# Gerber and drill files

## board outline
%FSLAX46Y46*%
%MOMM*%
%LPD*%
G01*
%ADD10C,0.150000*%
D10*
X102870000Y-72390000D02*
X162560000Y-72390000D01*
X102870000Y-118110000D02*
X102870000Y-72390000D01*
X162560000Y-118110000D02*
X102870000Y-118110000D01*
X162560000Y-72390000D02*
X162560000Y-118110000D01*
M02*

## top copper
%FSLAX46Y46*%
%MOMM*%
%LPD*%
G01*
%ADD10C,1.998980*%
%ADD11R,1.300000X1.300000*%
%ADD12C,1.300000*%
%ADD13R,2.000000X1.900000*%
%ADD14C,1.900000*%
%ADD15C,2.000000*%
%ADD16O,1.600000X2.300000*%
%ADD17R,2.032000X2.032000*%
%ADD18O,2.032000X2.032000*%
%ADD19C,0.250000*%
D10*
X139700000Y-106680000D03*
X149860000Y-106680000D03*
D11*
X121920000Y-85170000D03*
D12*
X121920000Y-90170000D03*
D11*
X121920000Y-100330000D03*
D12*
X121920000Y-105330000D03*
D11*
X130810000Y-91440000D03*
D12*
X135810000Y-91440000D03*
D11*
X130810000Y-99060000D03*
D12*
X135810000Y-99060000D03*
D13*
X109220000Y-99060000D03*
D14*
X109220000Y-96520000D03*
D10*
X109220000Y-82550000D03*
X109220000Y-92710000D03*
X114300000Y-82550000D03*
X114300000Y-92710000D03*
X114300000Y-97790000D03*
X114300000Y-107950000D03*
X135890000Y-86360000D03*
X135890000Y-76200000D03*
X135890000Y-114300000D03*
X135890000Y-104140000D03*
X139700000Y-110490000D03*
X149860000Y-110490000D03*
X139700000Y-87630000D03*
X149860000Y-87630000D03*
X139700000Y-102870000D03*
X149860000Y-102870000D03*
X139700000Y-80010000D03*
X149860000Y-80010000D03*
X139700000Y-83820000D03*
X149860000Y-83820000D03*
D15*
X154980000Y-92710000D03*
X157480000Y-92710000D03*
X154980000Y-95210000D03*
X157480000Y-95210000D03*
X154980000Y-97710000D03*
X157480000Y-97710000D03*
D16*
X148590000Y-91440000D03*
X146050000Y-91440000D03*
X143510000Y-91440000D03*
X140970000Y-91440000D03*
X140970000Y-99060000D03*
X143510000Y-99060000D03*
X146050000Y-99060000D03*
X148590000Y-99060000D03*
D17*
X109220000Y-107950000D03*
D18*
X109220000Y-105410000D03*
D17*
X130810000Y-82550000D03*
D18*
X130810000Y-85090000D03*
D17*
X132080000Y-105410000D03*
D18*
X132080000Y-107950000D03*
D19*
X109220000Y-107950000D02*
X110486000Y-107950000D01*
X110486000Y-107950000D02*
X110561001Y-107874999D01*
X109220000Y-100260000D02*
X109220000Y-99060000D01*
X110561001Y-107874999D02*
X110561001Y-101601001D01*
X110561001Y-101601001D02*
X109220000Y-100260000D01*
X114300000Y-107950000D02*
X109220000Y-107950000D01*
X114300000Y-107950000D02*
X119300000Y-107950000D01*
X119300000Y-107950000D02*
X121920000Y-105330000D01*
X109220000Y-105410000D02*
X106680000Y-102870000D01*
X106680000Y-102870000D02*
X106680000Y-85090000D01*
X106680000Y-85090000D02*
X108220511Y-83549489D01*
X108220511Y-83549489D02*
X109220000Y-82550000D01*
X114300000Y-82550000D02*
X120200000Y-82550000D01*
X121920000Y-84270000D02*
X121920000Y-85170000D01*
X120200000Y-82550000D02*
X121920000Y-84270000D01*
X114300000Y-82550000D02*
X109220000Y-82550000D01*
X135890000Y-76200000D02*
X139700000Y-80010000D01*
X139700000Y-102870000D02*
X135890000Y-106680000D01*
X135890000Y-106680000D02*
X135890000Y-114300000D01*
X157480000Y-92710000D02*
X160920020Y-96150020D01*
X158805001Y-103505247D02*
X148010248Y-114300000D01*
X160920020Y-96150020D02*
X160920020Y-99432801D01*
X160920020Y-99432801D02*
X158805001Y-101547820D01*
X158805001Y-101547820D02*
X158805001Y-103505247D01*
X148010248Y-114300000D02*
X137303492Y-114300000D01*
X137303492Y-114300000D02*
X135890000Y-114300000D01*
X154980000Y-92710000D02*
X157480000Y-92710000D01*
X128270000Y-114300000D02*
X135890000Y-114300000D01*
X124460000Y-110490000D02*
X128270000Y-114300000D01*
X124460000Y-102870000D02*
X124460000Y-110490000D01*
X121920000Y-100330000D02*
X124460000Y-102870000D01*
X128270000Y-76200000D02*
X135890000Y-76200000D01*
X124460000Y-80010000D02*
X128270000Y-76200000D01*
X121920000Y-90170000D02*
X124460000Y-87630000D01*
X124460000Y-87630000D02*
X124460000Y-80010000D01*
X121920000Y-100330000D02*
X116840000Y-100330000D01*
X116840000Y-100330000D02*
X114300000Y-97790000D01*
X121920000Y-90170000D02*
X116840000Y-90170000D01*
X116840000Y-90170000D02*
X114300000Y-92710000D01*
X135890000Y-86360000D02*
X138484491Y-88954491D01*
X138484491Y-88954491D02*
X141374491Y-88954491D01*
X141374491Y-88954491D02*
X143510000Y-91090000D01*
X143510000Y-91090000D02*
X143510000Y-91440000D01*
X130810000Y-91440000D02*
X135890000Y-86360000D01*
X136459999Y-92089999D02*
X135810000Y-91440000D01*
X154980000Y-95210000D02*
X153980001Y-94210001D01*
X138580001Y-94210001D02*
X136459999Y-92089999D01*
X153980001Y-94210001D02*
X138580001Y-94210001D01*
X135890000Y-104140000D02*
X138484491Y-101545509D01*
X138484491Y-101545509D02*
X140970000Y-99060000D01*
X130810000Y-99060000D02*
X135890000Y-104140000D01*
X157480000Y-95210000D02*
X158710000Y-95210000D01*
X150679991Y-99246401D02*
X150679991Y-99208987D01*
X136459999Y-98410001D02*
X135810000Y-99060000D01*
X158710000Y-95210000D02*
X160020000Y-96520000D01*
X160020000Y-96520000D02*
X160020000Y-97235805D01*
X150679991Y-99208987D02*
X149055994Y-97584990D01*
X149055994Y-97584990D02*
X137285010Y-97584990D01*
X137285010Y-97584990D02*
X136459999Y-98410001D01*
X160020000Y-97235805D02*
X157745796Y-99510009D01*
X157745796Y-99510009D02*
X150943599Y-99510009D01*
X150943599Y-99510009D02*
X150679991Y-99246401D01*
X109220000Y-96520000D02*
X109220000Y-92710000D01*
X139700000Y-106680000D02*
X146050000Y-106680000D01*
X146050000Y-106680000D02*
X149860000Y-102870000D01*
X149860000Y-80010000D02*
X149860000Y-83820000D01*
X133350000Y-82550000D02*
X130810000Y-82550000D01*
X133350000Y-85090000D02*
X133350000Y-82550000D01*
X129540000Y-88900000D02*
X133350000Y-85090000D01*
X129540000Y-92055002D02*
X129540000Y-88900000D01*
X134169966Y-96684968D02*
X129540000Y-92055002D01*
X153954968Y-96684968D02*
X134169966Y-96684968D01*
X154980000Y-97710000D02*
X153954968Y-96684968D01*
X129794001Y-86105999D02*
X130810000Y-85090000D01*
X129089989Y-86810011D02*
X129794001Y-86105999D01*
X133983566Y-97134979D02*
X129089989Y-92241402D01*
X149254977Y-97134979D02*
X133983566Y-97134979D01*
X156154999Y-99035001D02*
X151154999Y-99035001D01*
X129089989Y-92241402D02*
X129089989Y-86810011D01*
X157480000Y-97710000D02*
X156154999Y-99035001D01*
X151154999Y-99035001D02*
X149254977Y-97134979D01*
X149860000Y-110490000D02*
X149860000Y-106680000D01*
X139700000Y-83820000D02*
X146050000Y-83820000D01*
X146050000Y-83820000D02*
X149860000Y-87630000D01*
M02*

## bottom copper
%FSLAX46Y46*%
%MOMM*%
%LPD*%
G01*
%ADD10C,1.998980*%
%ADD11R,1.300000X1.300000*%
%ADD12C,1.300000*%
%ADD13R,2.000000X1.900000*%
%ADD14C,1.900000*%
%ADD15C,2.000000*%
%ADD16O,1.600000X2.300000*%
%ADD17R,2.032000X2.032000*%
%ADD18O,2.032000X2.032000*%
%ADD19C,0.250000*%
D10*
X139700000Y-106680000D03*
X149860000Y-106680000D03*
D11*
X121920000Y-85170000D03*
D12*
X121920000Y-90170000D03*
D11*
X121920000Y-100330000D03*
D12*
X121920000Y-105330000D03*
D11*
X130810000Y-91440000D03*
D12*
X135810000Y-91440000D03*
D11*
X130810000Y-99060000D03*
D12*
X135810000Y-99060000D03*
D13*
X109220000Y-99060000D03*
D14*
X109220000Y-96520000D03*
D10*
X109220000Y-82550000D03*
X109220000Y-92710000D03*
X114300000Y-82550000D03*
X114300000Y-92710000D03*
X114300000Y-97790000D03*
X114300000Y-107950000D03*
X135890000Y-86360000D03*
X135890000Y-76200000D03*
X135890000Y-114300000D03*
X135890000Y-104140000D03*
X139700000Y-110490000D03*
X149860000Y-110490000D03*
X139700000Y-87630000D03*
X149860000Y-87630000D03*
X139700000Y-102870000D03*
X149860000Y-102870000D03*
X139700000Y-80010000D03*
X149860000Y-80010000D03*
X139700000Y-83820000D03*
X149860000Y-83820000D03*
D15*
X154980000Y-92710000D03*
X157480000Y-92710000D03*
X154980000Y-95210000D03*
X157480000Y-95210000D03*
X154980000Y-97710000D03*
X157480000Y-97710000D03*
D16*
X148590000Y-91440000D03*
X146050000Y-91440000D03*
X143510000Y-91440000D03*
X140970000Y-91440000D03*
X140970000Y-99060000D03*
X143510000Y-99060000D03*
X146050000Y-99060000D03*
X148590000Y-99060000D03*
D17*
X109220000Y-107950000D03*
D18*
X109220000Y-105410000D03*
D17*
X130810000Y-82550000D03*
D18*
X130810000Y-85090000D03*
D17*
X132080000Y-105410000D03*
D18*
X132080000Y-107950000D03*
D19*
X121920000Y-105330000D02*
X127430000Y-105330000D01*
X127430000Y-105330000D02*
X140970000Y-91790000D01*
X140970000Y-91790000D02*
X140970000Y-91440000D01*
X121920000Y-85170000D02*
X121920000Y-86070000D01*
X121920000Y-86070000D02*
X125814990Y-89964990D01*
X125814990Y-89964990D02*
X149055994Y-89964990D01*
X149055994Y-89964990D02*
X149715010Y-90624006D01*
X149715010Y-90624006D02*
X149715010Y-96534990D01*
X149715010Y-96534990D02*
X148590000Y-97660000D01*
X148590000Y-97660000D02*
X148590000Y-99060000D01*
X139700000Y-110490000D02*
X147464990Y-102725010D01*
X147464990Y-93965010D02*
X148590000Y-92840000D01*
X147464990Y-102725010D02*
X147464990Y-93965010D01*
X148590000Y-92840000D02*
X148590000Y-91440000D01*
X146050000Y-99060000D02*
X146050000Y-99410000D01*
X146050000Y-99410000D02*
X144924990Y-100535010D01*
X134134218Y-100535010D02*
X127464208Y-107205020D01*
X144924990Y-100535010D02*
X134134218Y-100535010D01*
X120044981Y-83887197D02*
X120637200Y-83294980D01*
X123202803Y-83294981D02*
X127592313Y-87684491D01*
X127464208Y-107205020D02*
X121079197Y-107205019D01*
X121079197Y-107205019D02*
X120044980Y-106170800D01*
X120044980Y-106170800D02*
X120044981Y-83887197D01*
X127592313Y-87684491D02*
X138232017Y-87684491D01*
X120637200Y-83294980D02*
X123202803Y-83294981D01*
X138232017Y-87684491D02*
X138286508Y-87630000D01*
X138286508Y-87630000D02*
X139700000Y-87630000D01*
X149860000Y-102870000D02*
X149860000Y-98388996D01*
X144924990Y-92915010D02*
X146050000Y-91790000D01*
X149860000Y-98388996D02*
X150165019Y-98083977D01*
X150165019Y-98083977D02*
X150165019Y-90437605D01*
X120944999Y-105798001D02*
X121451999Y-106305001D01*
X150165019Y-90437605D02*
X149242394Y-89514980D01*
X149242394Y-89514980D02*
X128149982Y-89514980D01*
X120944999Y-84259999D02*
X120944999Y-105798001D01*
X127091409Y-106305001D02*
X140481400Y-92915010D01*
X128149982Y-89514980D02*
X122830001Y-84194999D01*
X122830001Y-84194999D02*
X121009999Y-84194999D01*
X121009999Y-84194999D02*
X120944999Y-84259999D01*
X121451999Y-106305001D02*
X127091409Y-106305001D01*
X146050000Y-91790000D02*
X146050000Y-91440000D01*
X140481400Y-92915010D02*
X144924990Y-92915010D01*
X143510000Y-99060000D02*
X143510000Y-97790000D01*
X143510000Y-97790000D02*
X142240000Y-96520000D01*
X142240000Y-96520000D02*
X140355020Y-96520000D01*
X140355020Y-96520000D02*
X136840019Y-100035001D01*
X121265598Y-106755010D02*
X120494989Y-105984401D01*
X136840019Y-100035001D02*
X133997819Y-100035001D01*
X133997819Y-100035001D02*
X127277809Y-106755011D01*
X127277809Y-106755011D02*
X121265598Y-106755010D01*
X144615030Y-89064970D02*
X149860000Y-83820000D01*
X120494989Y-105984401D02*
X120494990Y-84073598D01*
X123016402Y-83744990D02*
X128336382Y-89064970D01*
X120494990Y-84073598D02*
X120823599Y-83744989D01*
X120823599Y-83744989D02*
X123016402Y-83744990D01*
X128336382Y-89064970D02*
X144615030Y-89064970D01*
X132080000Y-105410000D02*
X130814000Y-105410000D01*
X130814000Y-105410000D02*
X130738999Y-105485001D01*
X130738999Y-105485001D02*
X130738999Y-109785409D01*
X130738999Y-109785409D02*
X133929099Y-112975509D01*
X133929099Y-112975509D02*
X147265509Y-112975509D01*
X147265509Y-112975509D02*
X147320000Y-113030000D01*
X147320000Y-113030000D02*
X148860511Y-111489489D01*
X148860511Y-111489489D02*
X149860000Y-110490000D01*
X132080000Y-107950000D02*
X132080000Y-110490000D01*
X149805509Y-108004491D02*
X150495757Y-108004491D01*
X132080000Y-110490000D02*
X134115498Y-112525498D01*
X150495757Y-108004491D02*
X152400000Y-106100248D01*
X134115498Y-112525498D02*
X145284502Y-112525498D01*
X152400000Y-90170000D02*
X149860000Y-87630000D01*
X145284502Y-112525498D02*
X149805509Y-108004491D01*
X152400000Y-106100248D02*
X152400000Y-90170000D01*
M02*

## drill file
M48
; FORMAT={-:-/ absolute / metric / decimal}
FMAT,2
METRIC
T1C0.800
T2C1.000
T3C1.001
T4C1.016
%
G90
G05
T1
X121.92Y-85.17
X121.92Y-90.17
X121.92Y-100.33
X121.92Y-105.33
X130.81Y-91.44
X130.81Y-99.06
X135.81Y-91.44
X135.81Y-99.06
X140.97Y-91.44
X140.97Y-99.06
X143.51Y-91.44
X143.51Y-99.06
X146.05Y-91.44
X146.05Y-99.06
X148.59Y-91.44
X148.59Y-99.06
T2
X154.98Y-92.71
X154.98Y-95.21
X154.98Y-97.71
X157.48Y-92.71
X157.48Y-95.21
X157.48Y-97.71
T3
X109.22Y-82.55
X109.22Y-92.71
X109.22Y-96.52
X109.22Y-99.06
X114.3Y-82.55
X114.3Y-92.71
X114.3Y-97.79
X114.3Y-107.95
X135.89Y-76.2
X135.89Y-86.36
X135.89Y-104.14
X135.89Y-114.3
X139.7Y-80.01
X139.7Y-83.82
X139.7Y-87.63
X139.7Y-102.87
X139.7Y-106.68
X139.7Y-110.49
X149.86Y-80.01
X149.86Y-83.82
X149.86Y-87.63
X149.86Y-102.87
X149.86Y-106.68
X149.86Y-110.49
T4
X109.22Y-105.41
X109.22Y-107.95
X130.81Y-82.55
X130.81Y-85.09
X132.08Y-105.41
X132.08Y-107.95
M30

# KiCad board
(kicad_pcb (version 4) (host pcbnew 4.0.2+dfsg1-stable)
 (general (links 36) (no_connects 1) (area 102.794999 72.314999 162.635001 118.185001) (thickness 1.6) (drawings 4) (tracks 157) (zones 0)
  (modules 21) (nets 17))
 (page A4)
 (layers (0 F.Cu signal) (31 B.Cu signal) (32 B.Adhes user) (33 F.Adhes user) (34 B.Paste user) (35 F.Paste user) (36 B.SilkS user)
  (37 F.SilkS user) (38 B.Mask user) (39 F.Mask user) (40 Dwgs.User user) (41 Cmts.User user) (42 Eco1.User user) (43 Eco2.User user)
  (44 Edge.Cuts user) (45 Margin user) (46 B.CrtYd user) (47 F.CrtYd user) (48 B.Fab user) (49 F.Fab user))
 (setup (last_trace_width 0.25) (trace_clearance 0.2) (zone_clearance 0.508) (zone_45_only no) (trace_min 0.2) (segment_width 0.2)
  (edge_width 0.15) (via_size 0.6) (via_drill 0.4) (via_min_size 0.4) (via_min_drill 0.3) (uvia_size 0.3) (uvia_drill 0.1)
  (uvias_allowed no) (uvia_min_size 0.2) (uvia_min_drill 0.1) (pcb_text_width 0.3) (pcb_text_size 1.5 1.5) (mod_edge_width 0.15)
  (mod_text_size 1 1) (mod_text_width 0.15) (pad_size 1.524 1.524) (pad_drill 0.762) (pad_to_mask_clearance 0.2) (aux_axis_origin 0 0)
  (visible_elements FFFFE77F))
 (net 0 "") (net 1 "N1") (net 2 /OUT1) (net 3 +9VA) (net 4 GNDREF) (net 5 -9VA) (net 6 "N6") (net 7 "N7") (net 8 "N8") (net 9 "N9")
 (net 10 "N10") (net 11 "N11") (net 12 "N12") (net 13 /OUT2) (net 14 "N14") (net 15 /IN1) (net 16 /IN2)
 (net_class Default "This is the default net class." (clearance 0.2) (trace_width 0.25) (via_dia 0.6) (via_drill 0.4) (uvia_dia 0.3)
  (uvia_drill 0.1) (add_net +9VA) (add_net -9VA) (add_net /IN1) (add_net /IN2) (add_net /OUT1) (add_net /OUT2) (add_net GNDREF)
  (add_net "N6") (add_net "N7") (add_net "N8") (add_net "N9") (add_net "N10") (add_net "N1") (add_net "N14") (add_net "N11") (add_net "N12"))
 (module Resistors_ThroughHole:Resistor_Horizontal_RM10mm (layer F.Cu) (at 139.7 106.68)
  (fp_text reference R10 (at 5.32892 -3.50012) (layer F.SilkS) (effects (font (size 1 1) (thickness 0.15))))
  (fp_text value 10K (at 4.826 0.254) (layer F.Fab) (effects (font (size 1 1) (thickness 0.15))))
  (pad 1 thru_hole circle (at 0 0) (size 1.99898 1.99898) (drill 1.00076) (layers *.Cu *.SilkS *.Mask) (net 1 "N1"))
  (pad 2 thru_hole circle (at 10.16 0) (size 1.99898 1.99898) (drill 1.00076) (layers *.Cu *.SilkS *.Mask) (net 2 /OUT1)))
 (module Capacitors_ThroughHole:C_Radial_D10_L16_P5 (layer F.Cu) (at 121.92 85.17 270)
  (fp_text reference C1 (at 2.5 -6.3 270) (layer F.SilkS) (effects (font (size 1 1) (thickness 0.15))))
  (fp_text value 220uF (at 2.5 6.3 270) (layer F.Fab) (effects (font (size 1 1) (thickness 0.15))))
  (pad 1 thru_hole rect (at 0 0 270) (size 1.3 1.3) (drill 0.8) (layers *.Cu *.Mask F.SilkS) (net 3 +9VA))
  (pad 2 thru_hole circle (at 5 0 270) (size 1.3 1.3) (drill 0.8) (layers *.Cu *.Mask F.SilkS) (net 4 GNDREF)))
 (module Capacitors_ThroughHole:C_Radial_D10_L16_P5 (layer F.Cu) (at 121.92 100.33 270)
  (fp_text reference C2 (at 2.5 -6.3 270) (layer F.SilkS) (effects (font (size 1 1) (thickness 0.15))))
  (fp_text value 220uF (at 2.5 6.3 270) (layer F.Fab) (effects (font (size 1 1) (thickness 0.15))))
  (pad 1 thru_hole rect (at 0 0 270) (size 1.3 1.3) (drill 0.8) (layers *.Cu *.Mask F.SilkS) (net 4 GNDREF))
  (pad 2 thru_hole circle (at 5 0 270) (size 1.3 1.3) (drill 0.8) (layers *.Cu *.Mask F.SilkS) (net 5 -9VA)))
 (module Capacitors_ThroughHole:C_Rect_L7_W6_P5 (layer F.Cu) (at 130.81 91.44)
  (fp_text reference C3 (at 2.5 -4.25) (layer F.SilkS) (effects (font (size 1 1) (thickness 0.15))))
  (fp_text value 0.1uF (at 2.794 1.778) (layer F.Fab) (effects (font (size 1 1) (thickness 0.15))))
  (pad 1 thru_hole rect (at 0 0) (size 1.3 1.3) (drill 0.8) (layers *.Cu *.Mask F.SilkS) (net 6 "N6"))
  (pad 2 thru_hole circle (at 5 0) (size 1.3 1.3) (drill 0.8) (layers *.Cu *.Mask F.SilkS) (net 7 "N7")))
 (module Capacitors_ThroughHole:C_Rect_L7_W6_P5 (layer F.Cu) (at 130.81 99.06)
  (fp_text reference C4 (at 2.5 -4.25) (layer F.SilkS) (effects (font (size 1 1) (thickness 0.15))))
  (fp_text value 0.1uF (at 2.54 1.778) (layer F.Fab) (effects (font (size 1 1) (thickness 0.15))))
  (pad 1 thru_hole rect (at 0 0) (size 1.3 1.3) (drill 0.8) (layers *.Cu *.Mask F.SilkS) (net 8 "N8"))
  (pad 2 thru_hole circle (at 5 0) (size 1.3 1.3) (drill 0.8) (layers *.Cu *.Mask F.SilkS) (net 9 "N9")))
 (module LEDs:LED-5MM (layer F.Cu) (at 109.22 99.06 90)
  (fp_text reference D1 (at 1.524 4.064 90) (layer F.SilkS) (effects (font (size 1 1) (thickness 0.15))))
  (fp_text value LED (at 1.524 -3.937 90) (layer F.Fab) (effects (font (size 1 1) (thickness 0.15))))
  (pad 1 thru_hole rect (at 0 0 180) (size 2 1.9) (drill 1.00076) (layers *.Cu *.Mask F.SilkS) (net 5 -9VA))
  (pad 2 thru_hole circle (at 2.54 0 90) (size 1.9 1.9) (drill 1.00076) (layers *.Cu *.Mask F.SilkS) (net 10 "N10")))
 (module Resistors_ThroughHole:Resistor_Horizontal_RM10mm (layer F.Cu) (at 109.22 82.55 270)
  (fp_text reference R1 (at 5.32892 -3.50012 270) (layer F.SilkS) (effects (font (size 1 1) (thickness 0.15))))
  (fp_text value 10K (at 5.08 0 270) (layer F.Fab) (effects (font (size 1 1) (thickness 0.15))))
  (pad 1 thru_hole circle (at 0 0 270) (size 1.99898 1.99898) (drill 1.00076) (layers *.Cu *.SilkS *.Mask) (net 3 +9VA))
  (pad 2 thru_hole circle (at 10.16 0 270) (size 1.99898 1.99898) (drill 1.00076) (layers *.Cu *.SilkS *.Mask) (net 10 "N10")))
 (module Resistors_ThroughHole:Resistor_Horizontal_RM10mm (layer F.Cu) (at 114.3 82.55 270)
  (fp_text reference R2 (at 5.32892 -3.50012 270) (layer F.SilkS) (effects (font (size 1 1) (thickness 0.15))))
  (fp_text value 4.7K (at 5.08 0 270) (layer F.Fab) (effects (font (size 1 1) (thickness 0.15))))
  (pad 1 thru_hole circle (at 0 0 270) (size 1.99898 1.99898) (drill 1.00076) (layers *.Cu *.SilkS *.Mask) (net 3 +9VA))
  (pad 2 thru_hole circle (at 10.16 0 270) (size 1.99898 1.99898) (drill 1.00076) (layers *.Cu *.SilkS *.Mask) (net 4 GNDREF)))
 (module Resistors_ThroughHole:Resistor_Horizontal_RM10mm (layer F.Cu) (at 114.3 97.79 270)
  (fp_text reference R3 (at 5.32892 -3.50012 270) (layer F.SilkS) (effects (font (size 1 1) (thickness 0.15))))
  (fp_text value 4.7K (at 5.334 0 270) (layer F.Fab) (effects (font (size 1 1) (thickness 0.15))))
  (pad 1 thru_hole circle (at 0 0 270) (size 1.99898 1.99898) (drill 1.00076) (layers *.Cu *.SilkS *.Mask) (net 4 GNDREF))
  (pad 2 thru_hole circle (at 10.16 0 270) (size 1.99898 1.99898) (drill 1.00076) (layers *.Cu *.SilkS *.Mask) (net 5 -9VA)))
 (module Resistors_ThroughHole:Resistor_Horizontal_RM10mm (layer F.Cu) (at 135.89 86.36 90)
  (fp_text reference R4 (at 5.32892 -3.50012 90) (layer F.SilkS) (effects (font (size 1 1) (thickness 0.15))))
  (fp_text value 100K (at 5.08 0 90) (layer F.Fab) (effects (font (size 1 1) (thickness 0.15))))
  (pad 1 thru_hole circle (at 0 0 90) (size 1.99898 1.99898) (drill 1.00076) (layers *.Cu *.SilkS *.Mask) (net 6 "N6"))
  (pad 2 thru_hole circle (at 10.16 0 90) (size 1.99898 1.99898) (drill 1.00076) (layers *.Cu *.SilkS *.Mask) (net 4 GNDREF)))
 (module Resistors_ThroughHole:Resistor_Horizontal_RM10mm (layer F.Cu) (at 135.89 114.3 90)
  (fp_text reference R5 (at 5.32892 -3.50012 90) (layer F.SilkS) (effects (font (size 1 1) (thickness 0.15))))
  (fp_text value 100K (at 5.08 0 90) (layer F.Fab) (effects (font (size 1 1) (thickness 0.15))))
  (pad 1 thru_hole circle (at 0 0 90) (size 1.99898 1.99898) (drill 1.00076) (layers *.Cu *.SilkS *.Mask) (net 4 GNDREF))
  (pad 2 thru_hole circle (at 10.16 0 90) (size 1.99898 1.99898) (drill 1.00076) (layers *.Cu *.SilkS *.Mask) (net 8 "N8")))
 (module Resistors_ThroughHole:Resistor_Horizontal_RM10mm (layer F.Cu) (at 139.7 110.49)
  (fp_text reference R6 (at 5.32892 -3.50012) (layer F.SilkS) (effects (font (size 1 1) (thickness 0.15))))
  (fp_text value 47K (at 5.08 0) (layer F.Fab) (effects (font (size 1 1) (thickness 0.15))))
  (pad 1 thru_hole circle (at 0 0) (size 1.99898 1.99898) (drill 1.00076) (layers *.Cu *.SilkS *.Mask) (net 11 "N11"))
  (pad 2 thru_hole circle (at 10.16 0) (size 1.99898 1.99898) (drill 1.00076) (layers *.Cu *.SilkS *.Mask) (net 2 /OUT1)))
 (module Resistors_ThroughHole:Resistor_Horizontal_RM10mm (layer F.Cu) (at 139.7 87.63)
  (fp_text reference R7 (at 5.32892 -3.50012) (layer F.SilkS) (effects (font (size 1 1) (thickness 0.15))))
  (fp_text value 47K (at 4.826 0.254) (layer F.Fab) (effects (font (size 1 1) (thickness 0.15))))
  (pad 1 thru_hole circle (at 0 0) (size 1.99898 1.99898) (drill 1.00076) (layers *.Cu *.SilkS *.Mask) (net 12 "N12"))
  (pad 2 thru_hole circle (at 10.16 0) (size 1.99898 1.99898) (drill 1.00076) (layers *.Cu *.SilkS *.Mask) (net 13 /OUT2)))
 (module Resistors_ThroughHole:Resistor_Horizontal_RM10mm (layer F.Cu) (at 139.7 102.87)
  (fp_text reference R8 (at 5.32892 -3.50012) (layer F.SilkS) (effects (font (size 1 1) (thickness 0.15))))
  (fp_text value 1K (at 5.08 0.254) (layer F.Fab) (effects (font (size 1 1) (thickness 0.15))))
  (pad 1 thru_hole circle (at 0 0) (size 1.99898 1.99898) (drill 1.00076) (layers *.Cu *.SilkS *.Mask) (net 4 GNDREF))
  (pad 2 thru_hole circle (at 10.16 0) (size 1.99898 1.99898) (drill 1.00076) (layers *.Cu *.SilkS *.Mask) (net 1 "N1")))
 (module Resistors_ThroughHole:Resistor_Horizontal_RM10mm (layer F.Cu) (at 139.7 80.01)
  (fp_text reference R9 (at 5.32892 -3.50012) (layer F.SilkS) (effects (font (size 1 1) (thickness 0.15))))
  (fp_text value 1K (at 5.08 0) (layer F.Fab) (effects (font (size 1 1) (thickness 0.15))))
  (pad 1 thru_hole circle (at 0 0) (size 1.99898 1.99898) (drill 1.00076) (layers *.Cu *.SilkS *.Mask) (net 4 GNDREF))
  (pad 2 thru_hole circle (at 10.16 0) (size 1.99898 1.99898) (drill 1.00076) (layers *.Cu *.SilkS *.Mask) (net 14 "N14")))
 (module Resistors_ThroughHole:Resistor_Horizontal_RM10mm (layer F.Cu) (at 139.7 83.82)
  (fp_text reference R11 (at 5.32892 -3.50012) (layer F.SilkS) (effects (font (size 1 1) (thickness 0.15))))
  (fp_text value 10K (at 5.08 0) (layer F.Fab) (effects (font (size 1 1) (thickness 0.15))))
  (pad 1 thru_hole circle (at 0 0) (size 1.99898 1.99898) (drill 1.00076) (layers *.Cu *.SilkS *.Mask) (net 13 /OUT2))
  (pad 2 thru_hole circle (at 10.16 0) (size 1.99898 1.99898) (drill 1.00076) (layers *.Cu *.SilkS *.Mask) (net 14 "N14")))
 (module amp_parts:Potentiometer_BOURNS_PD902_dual (layer F.Cu) (at 162.48 95.21)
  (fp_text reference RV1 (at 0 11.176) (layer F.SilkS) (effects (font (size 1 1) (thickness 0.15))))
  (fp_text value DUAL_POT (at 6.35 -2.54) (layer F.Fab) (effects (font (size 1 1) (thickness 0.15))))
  (pad 3 thru_hole circle (at -7.5 -2.5) (size 2 2) (drill 1) (layers *.Cu *.Mask F.SilkS) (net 4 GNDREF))
  (pad 6 thru_hole circle (at -5 -2.5) (size 2 2) (drill 1) (layers *.Cu *.Mask F.SilkS) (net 4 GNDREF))
  (pad 2 thru_hole circle (at -7.5 0) (size 2 2) (drill 1) (layers *.Cu *.Mask F.SilkS) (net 7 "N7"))
  (pad 5 thru_hole circle (at -5 0) (size 2 2) (drill 1) (layers *.Cu *.Mask F.SilkS) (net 9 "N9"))
  (pad 1 thru_hole circle (at -7.5 2.5) (size 2 2) (drill 1) (layers *.Cu *.Mask F.SilkS) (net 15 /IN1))
  (pad 4 thru_hole circle (at -5 2.5) (size 2 2) (drill 1) (layers *.Cu *.Mask F.SilkS) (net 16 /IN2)))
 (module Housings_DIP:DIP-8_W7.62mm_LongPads (layer F.Cu) (at 148.59 91.44 270)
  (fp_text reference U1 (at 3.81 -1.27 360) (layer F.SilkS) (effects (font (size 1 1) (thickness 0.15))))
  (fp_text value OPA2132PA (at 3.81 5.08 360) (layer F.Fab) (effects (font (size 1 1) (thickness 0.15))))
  (pad 1 thru_hole oval (at 0 0 270) (size 2.3 1.6) (drill 0.8) (layers *.Cu *.Mask F.SilkS) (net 11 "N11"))
  (pad 2 thru_hole oval (at 0 2.54 270) (size 2.3 1.6) (drill 0.8) (layers *.Cu *.Mask F.SilkS) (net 1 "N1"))
  (pad 3 thru_hole oval (at 0 5.08 270) (size 2.3 1.6) (drill 0.8) (layers *.Cu *.Mask F.SilkS) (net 6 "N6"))
  (pad 4 thru_hole oval (at 0 7.62 270) (size 2.3 1.6) (drill 0.8) (layers *.Cu *.Mask F.SilkS) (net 5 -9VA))
  (pad 5 thru_hole oval (at 7.62 7.62 270) (size 2.3 1.6) (drill 0.8) (layers *.Cu *.Mask F.SilkS) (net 8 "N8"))
  (pad 6 thru_hole oval (at 7.62 5.08 270) (size 2.3 1.6) (drill 0.8) (layers *.Cu *.Mask F.SilkS) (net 14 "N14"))
  (pad 7 thru_hole oval (at 7.62 2.54 270) (size 2.3 1.6) (drill 0.8) (layers *.Cu *.Mask F.SilkS) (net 12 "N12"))
  (pad 8 thru_hole oval (at 7.62 0 270) (size 2.3 1.6) (drill 0.8) (layers *.Cu *.Mask F.SilkS) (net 3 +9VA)))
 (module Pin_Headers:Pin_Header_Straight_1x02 (layer F.Cu) (at 109.22 107.95 180)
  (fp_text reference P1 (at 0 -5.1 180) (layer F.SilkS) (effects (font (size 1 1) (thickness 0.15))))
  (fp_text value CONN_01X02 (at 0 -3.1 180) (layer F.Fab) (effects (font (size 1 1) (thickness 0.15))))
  (pad 1 thru_hole rect (at 0 0 180) (size 2.032 2.032) (drill 1.016) (layers *.Cu *.Mask F.SilkS) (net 5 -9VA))
  (pad 2 thru_hole oval (at 0 2.54 180) (size 2.032 2.032) (drill 1.016) (layers *.Cu *.Mask F.SilkS) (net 3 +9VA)))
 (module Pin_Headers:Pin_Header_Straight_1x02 (layer F.Cu) (at 130.81 82.55)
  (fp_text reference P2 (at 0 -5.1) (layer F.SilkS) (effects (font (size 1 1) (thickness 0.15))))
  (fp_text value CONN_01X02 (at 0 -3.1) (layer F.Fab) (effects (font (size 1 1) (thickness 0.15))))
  (pad 1 thru_hole rect (at 0 0) (size 2.032 2.032) (drill 1.016) (layers *.Cu *.Mask F.SilkS) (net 15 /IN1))
  (pad 2 thru_hole oval (at 0 2.54) (size 2.032 2.032) (drill 1.016) (layers *.Cu *.Mask F.SilkS) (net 16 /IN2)))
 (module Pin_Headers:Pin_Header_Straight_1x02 (layer F.Cu) (at 132.08 105.41)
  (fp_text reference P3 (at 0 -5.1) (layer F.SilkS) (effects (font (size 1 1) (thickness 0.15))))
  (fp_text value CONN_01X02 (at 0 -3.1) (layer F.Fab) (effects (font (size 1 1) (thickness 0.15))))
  (pad 1 thru_hole rect (at 0 0) (size 2.032 2.032) (drill 1.016) (layers *.Cu *.Mask F.SilkS) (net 2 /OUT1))
  (pad 2 thru_hole oval (at 0 2.54) (size 2.032 2.032) (drill 1.016) (layers *.Cu *.Mask F.SilkS) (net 13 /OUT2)))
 (gr_line (start 102.87 72.39) (end 162.56 72.39) (layer Edge.Cuts) (width 0.15))
 (gr_line (start 102.87 118.11) (end 102.87 72.39) (layer Edge.Cuts) (width 0.15))
 (gr_line (start 162.56 118.11) (end 102.87 118.11) (layer Edge.Cuts) (width 0.15))
 (gr_line (start 162.56 72.39) (end 162.56 118.11) (layer Edge.Cuts) (width 0.15))
 (segment (start 162.56 73.66) (end 162.56 118.11) (width 0.25) (layer Dwgs.User) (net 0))
 (segment (start 121.92 105.33) (end 127.43 105.33) (width 0.25) (layer B.Cu) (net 5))
 (segment (start 127.43 105.33) (end 140.97 91.79) (width 0.25) (layer B.Cu) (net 5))
 (segment (start 140.97 91.79) (end 140.97 91.44) (width 0.25) (layer B.Cu) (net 5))
 (segment (start 109.22 107.95) (end 110.486 107.95) (width 0.25) (layer F.Cu) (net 5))
 (segment (start 110.486 107.95) (end 110.561001 107.874999) (width 0.25) (layer F.Cu) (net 5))
 (segment (start 109.22 100.26) (end 109.22 99.06) (width 0.25) (layer F.Cu) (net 5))
 (segment (start 110.561001 107.874999) (end 110.561001 101.601001) (width 0.25) (layer F.Cu) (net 5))
 (segment (start 110.561001 101.601001) (end 109.22 100.26) (width 0.25) (layer F.Cu) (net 5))
 (segment (start 114.3 107.95) (end 109.22 107.95) (width 0.25) (layer F.Cu) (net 5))
 (segment (start 114.3 107.95) (end 119.3 107.95) (width 0.25) (layer F.Cu) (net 5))
 (segment (start 119.3 107.95) (end 121.92 105.33) (width 0.25) (layer F.Cu) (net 5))
 (segment (start 109.22 105.41) (end 106.68 102.87) (width 0.25) (layer F.Cu) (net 3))
 (segment (start 106.68 102.87) (end 106.68 85.09) (width 0.25) (layer F.Cu) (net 3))
 (segment (start 106.68 85.09) (end 108.220511 83.549489) (width 0.25) (layer F.Cu) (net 3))
 (segment (start 108.220511 83.549489) (end 109.22 82.55) (width 0.25) (layer F.Cu) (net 3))
 (segment (start 121.92 85.17) (end 121.92 86.07) (width 0.25) (layer B.Cu) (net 3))
 (segment (start 121.92 86.07) (end 125.81499 89.96499) (width 0.25) (layer B.Cu) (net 3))
 (segment (start 125.81499 89.96499) (end 149.055994 89.96499) (width 0.25) (layer B.Cu) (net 3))
 (segment (start 149.055994 89.96499) (end 149.71501 90.624006) (width 0.25) (layer B.Cu) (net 3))
 (segment (start 149.71501 90.624006) (end 149.71501 96.53499) (width 0.25) (layer B.Cu) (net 3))
 (segment (start 149.71501 96.53499) (end 148.59 97.66) (width 0.25) (layer B.Cu) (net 3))
 (segment (start 148.59 97.66) (end 148.59 99.06) (width 0.25) (layer B.Cu) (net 3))
 (segment (start 114.3 82.55) (end 120.2 82.55) (width 0.25) (layer F.Cu) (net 3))
 (segment (start 121.92 84.27) (end 121.92 85.17) (width 0.25) (layer F.Cu) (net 3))
 (segment (start 120.2 82.55) (end 121.92 84.27) (width 0.25) (layer F.Cu) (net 3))
 (segment (start 114.3 82.55) (end 109.22 82.55) (width 0.25) (layer F.Cu) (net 3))
 (segment (start 135.89 76.2) (end 139.7 80.01) (width 0.25) (layer F.Cu) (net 4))
 (segment (start 139.7 102.87) (end 135.89 106.68) (width 0.25) (layer F.Cu) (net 4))
 (segment (start 135.89 106.68) (end 135.89 114.3) (width 0.25) (layer F.Cu) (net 4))
 (segment (start 157.48 92.71) (end 160.92002 96.15002) (width 0.25) (layer F.Cu) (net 4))
 (segment (start 158.805001 103.505247) (end 148.010248 114.3) (width 0.25) (layer F.Cu) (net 4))
 (segment (start 160.92002 96.15002) (end 160.92002 99.432801) (width 0.25) (layer F.Cu) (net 4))
 (segment (start 160.92002 99.432801) (end 158.805001 101.54782) (width 0.25) (layer F.Cu) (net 4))
 (segment (start 158.805001 101.54782) (end 158.805001 103.505247) (width 0.25) (layer F.Cu) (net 4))
 (segment (start 148.010248 114.3) (end 137.303492 114.3) (width 0.25) (layer F.Cu) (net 4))
 (segment (start 137.303492 114.3) (end 135.89 114.3) (width 0.25) (layer F.Cu) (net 4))
 (segment (start 154.98 92.71) (end 157.48 92.71) (width 0.25) (layer F.Cu) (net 4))
 (segment (start 128.27 114.3) (end 135.89 114.3) (width 0.25) (layer F.Cu) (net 4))
 (segment (start 124.46 110.49) (end 128.27 114.3) (width 0.25) (layer F.Cu) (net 4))
 (segment (start 124.46 102.87) (end 124.46 110.49) (width 0.25) (layer F.Cu) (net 4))
 (segment (start 121.92 100.33) (end 124.46 102.87) (width 0.25) (layer F.Cu) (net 4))
 (segment (start 128.27 76.2) (end 135.89 76.2) (width 0.25) (layer F.Cu) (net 4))
 (segment (start 124.46 80.01) (end 128.27 76.2) (width 0.25) (layer F.Cu) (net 4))
 (segment (start 121.92 90.17) (end 124.46 87.63) (width 0.25) (layer F.Cu) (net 4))
 (segment (start 124.46 87.63) (end 124.46 80.01) (width 0.25) (layer F.Cu) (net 4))
 (segment (start 121.92 100.33) (end 116.84 100.33) (width 0.25) (layer F.Cu) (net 4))
 (segment (start 116.84 100.33) (end 114.3 97.79) (width 0.25) (layer F.Cu) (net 4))
 (segment (start 121.92 90.17) (end 116.84 90.17) (width 0.25) (layer F.Cu) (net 4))
 (segment (start 116.84 90.17) (end 114.3 92.71) (width 0.25) (layer F.Cu) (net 4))
 (segment (start 135.89 86.36) (end 138.484491 88.954491) (width 0.25) (layer F.Cu) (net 6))
 (segment (start 138.484491 88.954491) (end 141.374491 88.954491) (width 0.25) (layer F.Cu) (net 6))
 (segment (start 141.374491 88.954491) (end 143.51 91.09) (width 0.25) (layer F.Cu) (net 6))
 (segment (start 143.51 91.09) (end 143.51 91.44) (width 0.25) (layer F.Cu) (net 6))
 (segment (start 130.81 91.44) (end 135.89 86.36) (width 0.25) (layer F.Cu) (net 6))
 (segment (start 136.459999 92.089999) (end 135.81 91.44) (width 0.25) (layer F.Cu) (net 7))
 (segment (start 154.98 95.21) (end 153.980001 94.210001) (width 0.25) (layer F.Cu) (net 7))
 (segment (start 138.580001 94.210001) (end 136.459999 92.089999) (width 0.25) (layer F.Cu) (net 7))
 (segment (start 153.980001 94.210001) (end 138.580001 94.210001) (width 0.25) (layer F.Cu) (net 7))
 (segment (start 135.89 104.14) (end 138.484491 101.545509) (width 0.25) (layer F.Cu) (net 8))
 (segment (start 138.484491 101.545509) (end 140.97 99.06) (width 0.25) (layer F.Cu) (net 8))
 (segment (start 130.81 99.06) (end 135.89 104.14) (width 0.25) (layer F.Cu) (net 8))
 (segment (start 157.48 95.21) (end 158.71 95.21) (width 0.25) (layer F.Cu) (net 9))
 (segment (start 150.679991 99.246401) (end 150.679991 99.208987) (width 0.25) (layer F.Cu) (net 9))
 (segment (start 136.459999 98.410001) (end 135.81 99.06) (width 0.25) (layer F.Cu) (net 9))
 (segment (start 158.71 95.21) (end 160.02 96.52) (width 0.25) (layer F.Cu) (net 9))
 (segment (start 160.02 96.52) (end 160.02 97.235805) (width 0.25) (layer F.Cu) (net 9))
 (segment (start 150.679991 99.208987) (end 149.055994 97.58499) (width 0.25) (layer F.Cu) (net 9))
 (segment (start 149.055994 97.58499) (end 137.28501 97.58499) (width 0.25) (layer F.Cu) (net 9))
 (segment (start 137.28501 97.58499) (end 136.459999 98.410001) (width 0.25) (layer F.Cu) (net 9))
 (segment (start 160.02 97.235805) (end 157.745796 99.510009) (width 0.25) (layer F.Cu) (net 9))
 (segment (start 157.745796 99.510009) (end 150.943599 99.510009) (width 0.25) (layer F.Cu) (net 9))
 (segment (start 150.943599 99.510009) (end 150.679991 99.246401) (width 0.25) (layer F.Cu) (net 9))
 (segment (start 109.22 96.52) (end 109.22 92.71) (width 0.25) (layer F.Cu) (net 10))
 (segment (start 139.7 110.49) (end 147.46499 102.72501) (width 0.25) (layer B.Cu) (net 11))
 (segment (start 147.46499 93.96501) (end 148.59 92.84) (width 0.25) (layer B.Cu) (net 11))
 (segment (start 147.46499 102.72501) (end 147.46499 93.96501) (width 0.25) (layer B.Cu) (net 11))
 (segment (start 148.59 92.84) (end 148.59 91.44) (width 0.25) (layer B.Cu) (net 11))
 (segment (start 146.05 99.06) (end 146.05 99.41) (width 0.25) (layer B.Cu) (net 12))
 (segment (start 146.05 99.41) (end 144.92499 100.53501) (width 0.25) (layer B.Cu) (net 12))
 (segment (start 134.134218 100.53501) (end 127.464208 107.20502) (width 0.25) (layer B.Cu) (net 12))
 (segment (start 144.92499 100.53501) (end 134.134218 100.53501) (width 0.25) (layer B.Cu) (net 12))
 (segment (start 120.044981 83.887197) (end 120.6372 83.29498) (width 0.25) (layer B.Cu) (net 12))
 (segment (start 123.202803 83.294981) (end 127.592313 87.684491) (width 0.25) (layer B.Cu) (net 12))
 (segment (start 127.464208 107.20502) (end 121.079197 107.205019) (width 0.25) (layer B.Cu) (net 12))
 (segment (start 121.079197 107.205019) (end 120.04498 106.1708) (width 0.25) (layer B.Cu) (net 12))
 (segment (start 120.04498 106.1708) (end 120.044981 83.887197) (width 0.25) (layer B.Cu) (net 12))
 (segment (start 127.592313 87.684491) (end 138.232017 87.684491) (width 0.25) (layer B.Cu) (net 12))
 (segment (start 120.6372 83.29498) (end 123.202803 83.294981) (width 0.25) (layer B.Cu) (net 12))
 (segment (start 138.232017 87.684491) (end 138.286508 87.63) (width 0.25) (layer B.Cu) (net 12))
 (segment (start 138.286508 87.63) (end 139.7 87.63) (width 0.25) (layer B.Cu) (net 12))
 (segment (start 149.86 102.87) (end 149.86 98.388996) (width 0.25) (layer B.Cu) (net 1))
 (segment (start 144.92499 92.91501) (end 146.05 91.79) (width 0.25) (layer B.Cu) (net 1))
 (segment (start 149.86 98.388996) (end 150.165019 98.083977) (width 0.25) (layer B.Cu) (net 1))
 (segment (start 150.165019 98.083977) (end 150.165019 90.437605) (width 0.25) (layer B.Cu) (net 1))
 (segment (start 120.944999 105.798001) (end 121.451999 106.305001) (width 0.25) (layer B.Cu) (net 1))
 (segment (start 150.165019 90.437605) (end 149.242394 89.51498) (width 0.25) (layer B.Cu) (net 1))
 (segment (start 149.242394 89.51498) (end 128.149982 89.51498) (width 0.25) (layer B.Cu) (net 1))
 (segment (start 120.944999 84.259999) (end 120.944999 105.798001) (width 0.25) (layer B.Cu) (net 1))
 (segment (start 127.091409 106.305001) (end 140.4814 92.91501) (width 0.25) (layer B.Cu) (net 1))
 (segment (start 128.149982 89.51498) (end 122.830001 84.194999) (width 0.25) (layer B.Cu) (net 1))
 (segment (start 122.830001 84.194999) (end 121.009999 84.194999) (width 0.25) (layer B.Cu) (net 1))
 (segment (start 121.009999 84.194999) (end 120.944999 84.259999) (width 0.25) (layer B.Cu) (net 1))
 (segment (start 121.451999 106.305001) (end 127.091409 106.305001) (width 0.25) (layer B.Cu) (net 1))
 (segment (start 146.05 91.79) (end 146.05 91.44) (width 0.25) (layer B.Cu) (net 1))
 (segment (start 140.4814 92.91501) (end 144.92499 92.91501) (width 0.25) (layer B.Cu) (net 1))
 (segment (start 139.7 106.68) (end 146.05 106.68) (width 0.25) (layer F.Cu) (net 1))
 (segment (start 146.05 106.68) (end 149.86 102.87) (width 0.25) (layer F.Cu) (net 1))
 (segment (start 143.51 99.06) (end 143.51 97.79) (width 0.25) (layer B.Cu) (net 14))
 (segment (start 143.51 97.79) (end 142.24 96.52) (width 0.25) (layer B.Cu) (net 14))
 (segment (start 142.24 96.52) (end 140.35502 96.52) (width 0.25) (layer B.Cu) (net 14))
 (segment (start 140.35502 96.52) (end 136.840019 100.035001) (width 0.25) (layer B.Cu) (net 14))
 (segment (start 121.265598 106.75501) (end 120.494989 105.984401) (width 0.25) (layer B.Cu) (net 14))
 (segment (start 136.840019 100.035001) (end 133.997819 100.035001) (width 0.25) (layer B.Cu) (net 14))
 (segment (start 133.997819 100.035001) (end 127.277809 106.755011) (width 0.25) (layer B.Cu) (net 14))
 (segment (start 127.277809 106.755011) (end 121.265598 106.75501) (width 0.25) (layer B.Cu) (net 14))
 (segment (start 144.61503 89.06497) (end 149.86 83.82) (width 0.25) (layer B.Cu) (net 14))
 (segment (start 120.494989 105.984401) (end 120.49499 84.073598) (width 0.25) (layer B.Cu) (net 14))
 (segment (start 123.016402 83.74499) (end 128.336382 89.06497) (width 0.25) (layer B.Cu) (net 14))
 (segment (start 120.49499 84.073598) (end 120.823599 83.744989) (width 0.25) (layer B.Cu) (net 14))
 (segment (start 120.823599 83.744989) (end 123.016402 83.74499) (width 0.25) (layer B.Cu) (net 14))
 (segment (start 128.336382 89.06497) (end 144.61503 89.06497) (width 0.25) (layer B.Cu) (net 14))
 (segment (start 149.86 80.01) (end 149.86 83.82) (width 0.25) (layer F.Cu) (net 14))
 (segment (start 133.35 82.55) (end 130.81 82.55) (width 0.25) (layer F.Cu) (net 15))
 (segment (start 133.35 85.09) (end 133.35 82.55) (width 0.25) (layer F.Cu) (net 15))
 (segment (start 129.54 88.9) (end 133.35 85.09) (width 0.25) (layer F.Cu) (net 15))
 (segment (start 129.54 92.055002) (end 129.54 88.9) (width 0.25) (layer F.Cu) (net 15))
 (segment (start 134.169966 96.684968) (end 129.54 92.055002) (width 0.25) (layer F.Cu) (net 15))
 (segment (start 153.954968 96.684968) (end 134.169966 96.684968) (width 0.25) (layer F.Cu) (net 15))
 (segment (start 154.98 97.71) (end 153.954968 96.684968) (width 0.25) (layer F.Cu) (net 15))
 (segment (start 129.794001 86.105999) (end 130.81 85.09) (width 0.25) (layer F.Cu) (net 16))
 (segment (start 129.089989 86.810011) (end 129.794001 86.105999) (width 0.25) (layer F.Cu) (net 16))
 (segment (start 133.983566 97.134979) (end 129.089989 92.241402) (width 0.25) (layer F.Cu) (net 16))
 (segment (start 149.254977 97.134979) (end 133.983566 97.134979) (width 0.25) (layer F.Cu) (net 16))
 (segment (start 156.154999 99.035001) (end 151.154999 99.035001) (width 0.25) (layer F.Cu) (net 16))
 (segment (start 129.089989 92.241402) (end 129.089989 86.810011) (width 0.25) (layer F.Cu) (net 16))
 (segment (start 157.48 97.71) (end 156.154999 99.035001) (width 0.25) (layer F.Cu) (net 16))
 (segment (start 151.154999 99.035001) (end 149.254977 97.134979) (width 0.25) (layer F.Cu) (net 16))
 (segment (start 132.08 105.41) (end 130.814 105.41) (width 0.25) (layer B.Cu) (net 2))
 (segment (start 130.814 105.41) (end 130.738999 105.485001) (width 0.25) (layer B.Cu) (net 2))
 (segment (start 130.738999 105.485001) (end 130.738999 109.785409) (width 0.25) (layer B.Cu) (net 2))
 (segment (start 130.738999 109.785409) (end 133.929099 112.975509) (width 0.25) (layer B.Cu) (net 2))
 (segment (start 133.929099 112.975509) (end 147.265509 112.975509) (width 0.25) (layer B.Cu) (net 2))
 (segment (start 147.265509 112.975509) (end 147.32 113.03) (width 0.25) (layer B.Cu) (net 2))
 (segment (start 147.32 113.03) (end 148.860511 111.489489) (width 0.25) (layer B.Cu) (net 2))
 (segment (start 148.860511 111.489489) (end 149.86 110.49) (width 0.25) (layer B.Cu) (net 2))
 (segment (start 149.86 110.49) (end 149.86 106.68) (width 0.25) (layer F.Cu) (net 2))
 (segment (start 132.08 107.95) (end 132.08 110.49) (width 0.25) (layer B.Cu) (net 13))
 (segment (start 149.805509 108.004491) (end 150.495757 108.004491) (width 0.25) (layer B.Cu) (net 13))
 (segment (start 132.08 110.49) (end 134.115498 112.525498) (width 0.25) (layer B.Cu) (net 13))
 (segment (start 150.495757 108.004491) (end 152.4 106.100248) (width 0.25) (layer B.Cu) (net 13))
 (segment (start 134.115498 112.525498) (end 145.284502 112.525498) (width 0.25) (layer B.Cu) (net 13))
 (segment (start 152.4 90.17) (end 149.86 87.63) (width 0.25) (layer B.Cu) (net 13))
 (segment (start 145.284502 112.525498) (end 149.805509 108.004491) (width 0.25) (layer B.Cu) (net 13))
 (segment (start 152.4 106.100248) (end 152.4 90.17) (width 0.25) (layer B.Cu) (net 13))
 (segment (start 139.7 83.82) (end 146.05 83.82) (width 0.25) (layer F.Cu) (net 13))
 (segment (start 146.05 83.82) (end 149.86 87.63) (width 0.25) (layer F.Cu) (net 13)))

